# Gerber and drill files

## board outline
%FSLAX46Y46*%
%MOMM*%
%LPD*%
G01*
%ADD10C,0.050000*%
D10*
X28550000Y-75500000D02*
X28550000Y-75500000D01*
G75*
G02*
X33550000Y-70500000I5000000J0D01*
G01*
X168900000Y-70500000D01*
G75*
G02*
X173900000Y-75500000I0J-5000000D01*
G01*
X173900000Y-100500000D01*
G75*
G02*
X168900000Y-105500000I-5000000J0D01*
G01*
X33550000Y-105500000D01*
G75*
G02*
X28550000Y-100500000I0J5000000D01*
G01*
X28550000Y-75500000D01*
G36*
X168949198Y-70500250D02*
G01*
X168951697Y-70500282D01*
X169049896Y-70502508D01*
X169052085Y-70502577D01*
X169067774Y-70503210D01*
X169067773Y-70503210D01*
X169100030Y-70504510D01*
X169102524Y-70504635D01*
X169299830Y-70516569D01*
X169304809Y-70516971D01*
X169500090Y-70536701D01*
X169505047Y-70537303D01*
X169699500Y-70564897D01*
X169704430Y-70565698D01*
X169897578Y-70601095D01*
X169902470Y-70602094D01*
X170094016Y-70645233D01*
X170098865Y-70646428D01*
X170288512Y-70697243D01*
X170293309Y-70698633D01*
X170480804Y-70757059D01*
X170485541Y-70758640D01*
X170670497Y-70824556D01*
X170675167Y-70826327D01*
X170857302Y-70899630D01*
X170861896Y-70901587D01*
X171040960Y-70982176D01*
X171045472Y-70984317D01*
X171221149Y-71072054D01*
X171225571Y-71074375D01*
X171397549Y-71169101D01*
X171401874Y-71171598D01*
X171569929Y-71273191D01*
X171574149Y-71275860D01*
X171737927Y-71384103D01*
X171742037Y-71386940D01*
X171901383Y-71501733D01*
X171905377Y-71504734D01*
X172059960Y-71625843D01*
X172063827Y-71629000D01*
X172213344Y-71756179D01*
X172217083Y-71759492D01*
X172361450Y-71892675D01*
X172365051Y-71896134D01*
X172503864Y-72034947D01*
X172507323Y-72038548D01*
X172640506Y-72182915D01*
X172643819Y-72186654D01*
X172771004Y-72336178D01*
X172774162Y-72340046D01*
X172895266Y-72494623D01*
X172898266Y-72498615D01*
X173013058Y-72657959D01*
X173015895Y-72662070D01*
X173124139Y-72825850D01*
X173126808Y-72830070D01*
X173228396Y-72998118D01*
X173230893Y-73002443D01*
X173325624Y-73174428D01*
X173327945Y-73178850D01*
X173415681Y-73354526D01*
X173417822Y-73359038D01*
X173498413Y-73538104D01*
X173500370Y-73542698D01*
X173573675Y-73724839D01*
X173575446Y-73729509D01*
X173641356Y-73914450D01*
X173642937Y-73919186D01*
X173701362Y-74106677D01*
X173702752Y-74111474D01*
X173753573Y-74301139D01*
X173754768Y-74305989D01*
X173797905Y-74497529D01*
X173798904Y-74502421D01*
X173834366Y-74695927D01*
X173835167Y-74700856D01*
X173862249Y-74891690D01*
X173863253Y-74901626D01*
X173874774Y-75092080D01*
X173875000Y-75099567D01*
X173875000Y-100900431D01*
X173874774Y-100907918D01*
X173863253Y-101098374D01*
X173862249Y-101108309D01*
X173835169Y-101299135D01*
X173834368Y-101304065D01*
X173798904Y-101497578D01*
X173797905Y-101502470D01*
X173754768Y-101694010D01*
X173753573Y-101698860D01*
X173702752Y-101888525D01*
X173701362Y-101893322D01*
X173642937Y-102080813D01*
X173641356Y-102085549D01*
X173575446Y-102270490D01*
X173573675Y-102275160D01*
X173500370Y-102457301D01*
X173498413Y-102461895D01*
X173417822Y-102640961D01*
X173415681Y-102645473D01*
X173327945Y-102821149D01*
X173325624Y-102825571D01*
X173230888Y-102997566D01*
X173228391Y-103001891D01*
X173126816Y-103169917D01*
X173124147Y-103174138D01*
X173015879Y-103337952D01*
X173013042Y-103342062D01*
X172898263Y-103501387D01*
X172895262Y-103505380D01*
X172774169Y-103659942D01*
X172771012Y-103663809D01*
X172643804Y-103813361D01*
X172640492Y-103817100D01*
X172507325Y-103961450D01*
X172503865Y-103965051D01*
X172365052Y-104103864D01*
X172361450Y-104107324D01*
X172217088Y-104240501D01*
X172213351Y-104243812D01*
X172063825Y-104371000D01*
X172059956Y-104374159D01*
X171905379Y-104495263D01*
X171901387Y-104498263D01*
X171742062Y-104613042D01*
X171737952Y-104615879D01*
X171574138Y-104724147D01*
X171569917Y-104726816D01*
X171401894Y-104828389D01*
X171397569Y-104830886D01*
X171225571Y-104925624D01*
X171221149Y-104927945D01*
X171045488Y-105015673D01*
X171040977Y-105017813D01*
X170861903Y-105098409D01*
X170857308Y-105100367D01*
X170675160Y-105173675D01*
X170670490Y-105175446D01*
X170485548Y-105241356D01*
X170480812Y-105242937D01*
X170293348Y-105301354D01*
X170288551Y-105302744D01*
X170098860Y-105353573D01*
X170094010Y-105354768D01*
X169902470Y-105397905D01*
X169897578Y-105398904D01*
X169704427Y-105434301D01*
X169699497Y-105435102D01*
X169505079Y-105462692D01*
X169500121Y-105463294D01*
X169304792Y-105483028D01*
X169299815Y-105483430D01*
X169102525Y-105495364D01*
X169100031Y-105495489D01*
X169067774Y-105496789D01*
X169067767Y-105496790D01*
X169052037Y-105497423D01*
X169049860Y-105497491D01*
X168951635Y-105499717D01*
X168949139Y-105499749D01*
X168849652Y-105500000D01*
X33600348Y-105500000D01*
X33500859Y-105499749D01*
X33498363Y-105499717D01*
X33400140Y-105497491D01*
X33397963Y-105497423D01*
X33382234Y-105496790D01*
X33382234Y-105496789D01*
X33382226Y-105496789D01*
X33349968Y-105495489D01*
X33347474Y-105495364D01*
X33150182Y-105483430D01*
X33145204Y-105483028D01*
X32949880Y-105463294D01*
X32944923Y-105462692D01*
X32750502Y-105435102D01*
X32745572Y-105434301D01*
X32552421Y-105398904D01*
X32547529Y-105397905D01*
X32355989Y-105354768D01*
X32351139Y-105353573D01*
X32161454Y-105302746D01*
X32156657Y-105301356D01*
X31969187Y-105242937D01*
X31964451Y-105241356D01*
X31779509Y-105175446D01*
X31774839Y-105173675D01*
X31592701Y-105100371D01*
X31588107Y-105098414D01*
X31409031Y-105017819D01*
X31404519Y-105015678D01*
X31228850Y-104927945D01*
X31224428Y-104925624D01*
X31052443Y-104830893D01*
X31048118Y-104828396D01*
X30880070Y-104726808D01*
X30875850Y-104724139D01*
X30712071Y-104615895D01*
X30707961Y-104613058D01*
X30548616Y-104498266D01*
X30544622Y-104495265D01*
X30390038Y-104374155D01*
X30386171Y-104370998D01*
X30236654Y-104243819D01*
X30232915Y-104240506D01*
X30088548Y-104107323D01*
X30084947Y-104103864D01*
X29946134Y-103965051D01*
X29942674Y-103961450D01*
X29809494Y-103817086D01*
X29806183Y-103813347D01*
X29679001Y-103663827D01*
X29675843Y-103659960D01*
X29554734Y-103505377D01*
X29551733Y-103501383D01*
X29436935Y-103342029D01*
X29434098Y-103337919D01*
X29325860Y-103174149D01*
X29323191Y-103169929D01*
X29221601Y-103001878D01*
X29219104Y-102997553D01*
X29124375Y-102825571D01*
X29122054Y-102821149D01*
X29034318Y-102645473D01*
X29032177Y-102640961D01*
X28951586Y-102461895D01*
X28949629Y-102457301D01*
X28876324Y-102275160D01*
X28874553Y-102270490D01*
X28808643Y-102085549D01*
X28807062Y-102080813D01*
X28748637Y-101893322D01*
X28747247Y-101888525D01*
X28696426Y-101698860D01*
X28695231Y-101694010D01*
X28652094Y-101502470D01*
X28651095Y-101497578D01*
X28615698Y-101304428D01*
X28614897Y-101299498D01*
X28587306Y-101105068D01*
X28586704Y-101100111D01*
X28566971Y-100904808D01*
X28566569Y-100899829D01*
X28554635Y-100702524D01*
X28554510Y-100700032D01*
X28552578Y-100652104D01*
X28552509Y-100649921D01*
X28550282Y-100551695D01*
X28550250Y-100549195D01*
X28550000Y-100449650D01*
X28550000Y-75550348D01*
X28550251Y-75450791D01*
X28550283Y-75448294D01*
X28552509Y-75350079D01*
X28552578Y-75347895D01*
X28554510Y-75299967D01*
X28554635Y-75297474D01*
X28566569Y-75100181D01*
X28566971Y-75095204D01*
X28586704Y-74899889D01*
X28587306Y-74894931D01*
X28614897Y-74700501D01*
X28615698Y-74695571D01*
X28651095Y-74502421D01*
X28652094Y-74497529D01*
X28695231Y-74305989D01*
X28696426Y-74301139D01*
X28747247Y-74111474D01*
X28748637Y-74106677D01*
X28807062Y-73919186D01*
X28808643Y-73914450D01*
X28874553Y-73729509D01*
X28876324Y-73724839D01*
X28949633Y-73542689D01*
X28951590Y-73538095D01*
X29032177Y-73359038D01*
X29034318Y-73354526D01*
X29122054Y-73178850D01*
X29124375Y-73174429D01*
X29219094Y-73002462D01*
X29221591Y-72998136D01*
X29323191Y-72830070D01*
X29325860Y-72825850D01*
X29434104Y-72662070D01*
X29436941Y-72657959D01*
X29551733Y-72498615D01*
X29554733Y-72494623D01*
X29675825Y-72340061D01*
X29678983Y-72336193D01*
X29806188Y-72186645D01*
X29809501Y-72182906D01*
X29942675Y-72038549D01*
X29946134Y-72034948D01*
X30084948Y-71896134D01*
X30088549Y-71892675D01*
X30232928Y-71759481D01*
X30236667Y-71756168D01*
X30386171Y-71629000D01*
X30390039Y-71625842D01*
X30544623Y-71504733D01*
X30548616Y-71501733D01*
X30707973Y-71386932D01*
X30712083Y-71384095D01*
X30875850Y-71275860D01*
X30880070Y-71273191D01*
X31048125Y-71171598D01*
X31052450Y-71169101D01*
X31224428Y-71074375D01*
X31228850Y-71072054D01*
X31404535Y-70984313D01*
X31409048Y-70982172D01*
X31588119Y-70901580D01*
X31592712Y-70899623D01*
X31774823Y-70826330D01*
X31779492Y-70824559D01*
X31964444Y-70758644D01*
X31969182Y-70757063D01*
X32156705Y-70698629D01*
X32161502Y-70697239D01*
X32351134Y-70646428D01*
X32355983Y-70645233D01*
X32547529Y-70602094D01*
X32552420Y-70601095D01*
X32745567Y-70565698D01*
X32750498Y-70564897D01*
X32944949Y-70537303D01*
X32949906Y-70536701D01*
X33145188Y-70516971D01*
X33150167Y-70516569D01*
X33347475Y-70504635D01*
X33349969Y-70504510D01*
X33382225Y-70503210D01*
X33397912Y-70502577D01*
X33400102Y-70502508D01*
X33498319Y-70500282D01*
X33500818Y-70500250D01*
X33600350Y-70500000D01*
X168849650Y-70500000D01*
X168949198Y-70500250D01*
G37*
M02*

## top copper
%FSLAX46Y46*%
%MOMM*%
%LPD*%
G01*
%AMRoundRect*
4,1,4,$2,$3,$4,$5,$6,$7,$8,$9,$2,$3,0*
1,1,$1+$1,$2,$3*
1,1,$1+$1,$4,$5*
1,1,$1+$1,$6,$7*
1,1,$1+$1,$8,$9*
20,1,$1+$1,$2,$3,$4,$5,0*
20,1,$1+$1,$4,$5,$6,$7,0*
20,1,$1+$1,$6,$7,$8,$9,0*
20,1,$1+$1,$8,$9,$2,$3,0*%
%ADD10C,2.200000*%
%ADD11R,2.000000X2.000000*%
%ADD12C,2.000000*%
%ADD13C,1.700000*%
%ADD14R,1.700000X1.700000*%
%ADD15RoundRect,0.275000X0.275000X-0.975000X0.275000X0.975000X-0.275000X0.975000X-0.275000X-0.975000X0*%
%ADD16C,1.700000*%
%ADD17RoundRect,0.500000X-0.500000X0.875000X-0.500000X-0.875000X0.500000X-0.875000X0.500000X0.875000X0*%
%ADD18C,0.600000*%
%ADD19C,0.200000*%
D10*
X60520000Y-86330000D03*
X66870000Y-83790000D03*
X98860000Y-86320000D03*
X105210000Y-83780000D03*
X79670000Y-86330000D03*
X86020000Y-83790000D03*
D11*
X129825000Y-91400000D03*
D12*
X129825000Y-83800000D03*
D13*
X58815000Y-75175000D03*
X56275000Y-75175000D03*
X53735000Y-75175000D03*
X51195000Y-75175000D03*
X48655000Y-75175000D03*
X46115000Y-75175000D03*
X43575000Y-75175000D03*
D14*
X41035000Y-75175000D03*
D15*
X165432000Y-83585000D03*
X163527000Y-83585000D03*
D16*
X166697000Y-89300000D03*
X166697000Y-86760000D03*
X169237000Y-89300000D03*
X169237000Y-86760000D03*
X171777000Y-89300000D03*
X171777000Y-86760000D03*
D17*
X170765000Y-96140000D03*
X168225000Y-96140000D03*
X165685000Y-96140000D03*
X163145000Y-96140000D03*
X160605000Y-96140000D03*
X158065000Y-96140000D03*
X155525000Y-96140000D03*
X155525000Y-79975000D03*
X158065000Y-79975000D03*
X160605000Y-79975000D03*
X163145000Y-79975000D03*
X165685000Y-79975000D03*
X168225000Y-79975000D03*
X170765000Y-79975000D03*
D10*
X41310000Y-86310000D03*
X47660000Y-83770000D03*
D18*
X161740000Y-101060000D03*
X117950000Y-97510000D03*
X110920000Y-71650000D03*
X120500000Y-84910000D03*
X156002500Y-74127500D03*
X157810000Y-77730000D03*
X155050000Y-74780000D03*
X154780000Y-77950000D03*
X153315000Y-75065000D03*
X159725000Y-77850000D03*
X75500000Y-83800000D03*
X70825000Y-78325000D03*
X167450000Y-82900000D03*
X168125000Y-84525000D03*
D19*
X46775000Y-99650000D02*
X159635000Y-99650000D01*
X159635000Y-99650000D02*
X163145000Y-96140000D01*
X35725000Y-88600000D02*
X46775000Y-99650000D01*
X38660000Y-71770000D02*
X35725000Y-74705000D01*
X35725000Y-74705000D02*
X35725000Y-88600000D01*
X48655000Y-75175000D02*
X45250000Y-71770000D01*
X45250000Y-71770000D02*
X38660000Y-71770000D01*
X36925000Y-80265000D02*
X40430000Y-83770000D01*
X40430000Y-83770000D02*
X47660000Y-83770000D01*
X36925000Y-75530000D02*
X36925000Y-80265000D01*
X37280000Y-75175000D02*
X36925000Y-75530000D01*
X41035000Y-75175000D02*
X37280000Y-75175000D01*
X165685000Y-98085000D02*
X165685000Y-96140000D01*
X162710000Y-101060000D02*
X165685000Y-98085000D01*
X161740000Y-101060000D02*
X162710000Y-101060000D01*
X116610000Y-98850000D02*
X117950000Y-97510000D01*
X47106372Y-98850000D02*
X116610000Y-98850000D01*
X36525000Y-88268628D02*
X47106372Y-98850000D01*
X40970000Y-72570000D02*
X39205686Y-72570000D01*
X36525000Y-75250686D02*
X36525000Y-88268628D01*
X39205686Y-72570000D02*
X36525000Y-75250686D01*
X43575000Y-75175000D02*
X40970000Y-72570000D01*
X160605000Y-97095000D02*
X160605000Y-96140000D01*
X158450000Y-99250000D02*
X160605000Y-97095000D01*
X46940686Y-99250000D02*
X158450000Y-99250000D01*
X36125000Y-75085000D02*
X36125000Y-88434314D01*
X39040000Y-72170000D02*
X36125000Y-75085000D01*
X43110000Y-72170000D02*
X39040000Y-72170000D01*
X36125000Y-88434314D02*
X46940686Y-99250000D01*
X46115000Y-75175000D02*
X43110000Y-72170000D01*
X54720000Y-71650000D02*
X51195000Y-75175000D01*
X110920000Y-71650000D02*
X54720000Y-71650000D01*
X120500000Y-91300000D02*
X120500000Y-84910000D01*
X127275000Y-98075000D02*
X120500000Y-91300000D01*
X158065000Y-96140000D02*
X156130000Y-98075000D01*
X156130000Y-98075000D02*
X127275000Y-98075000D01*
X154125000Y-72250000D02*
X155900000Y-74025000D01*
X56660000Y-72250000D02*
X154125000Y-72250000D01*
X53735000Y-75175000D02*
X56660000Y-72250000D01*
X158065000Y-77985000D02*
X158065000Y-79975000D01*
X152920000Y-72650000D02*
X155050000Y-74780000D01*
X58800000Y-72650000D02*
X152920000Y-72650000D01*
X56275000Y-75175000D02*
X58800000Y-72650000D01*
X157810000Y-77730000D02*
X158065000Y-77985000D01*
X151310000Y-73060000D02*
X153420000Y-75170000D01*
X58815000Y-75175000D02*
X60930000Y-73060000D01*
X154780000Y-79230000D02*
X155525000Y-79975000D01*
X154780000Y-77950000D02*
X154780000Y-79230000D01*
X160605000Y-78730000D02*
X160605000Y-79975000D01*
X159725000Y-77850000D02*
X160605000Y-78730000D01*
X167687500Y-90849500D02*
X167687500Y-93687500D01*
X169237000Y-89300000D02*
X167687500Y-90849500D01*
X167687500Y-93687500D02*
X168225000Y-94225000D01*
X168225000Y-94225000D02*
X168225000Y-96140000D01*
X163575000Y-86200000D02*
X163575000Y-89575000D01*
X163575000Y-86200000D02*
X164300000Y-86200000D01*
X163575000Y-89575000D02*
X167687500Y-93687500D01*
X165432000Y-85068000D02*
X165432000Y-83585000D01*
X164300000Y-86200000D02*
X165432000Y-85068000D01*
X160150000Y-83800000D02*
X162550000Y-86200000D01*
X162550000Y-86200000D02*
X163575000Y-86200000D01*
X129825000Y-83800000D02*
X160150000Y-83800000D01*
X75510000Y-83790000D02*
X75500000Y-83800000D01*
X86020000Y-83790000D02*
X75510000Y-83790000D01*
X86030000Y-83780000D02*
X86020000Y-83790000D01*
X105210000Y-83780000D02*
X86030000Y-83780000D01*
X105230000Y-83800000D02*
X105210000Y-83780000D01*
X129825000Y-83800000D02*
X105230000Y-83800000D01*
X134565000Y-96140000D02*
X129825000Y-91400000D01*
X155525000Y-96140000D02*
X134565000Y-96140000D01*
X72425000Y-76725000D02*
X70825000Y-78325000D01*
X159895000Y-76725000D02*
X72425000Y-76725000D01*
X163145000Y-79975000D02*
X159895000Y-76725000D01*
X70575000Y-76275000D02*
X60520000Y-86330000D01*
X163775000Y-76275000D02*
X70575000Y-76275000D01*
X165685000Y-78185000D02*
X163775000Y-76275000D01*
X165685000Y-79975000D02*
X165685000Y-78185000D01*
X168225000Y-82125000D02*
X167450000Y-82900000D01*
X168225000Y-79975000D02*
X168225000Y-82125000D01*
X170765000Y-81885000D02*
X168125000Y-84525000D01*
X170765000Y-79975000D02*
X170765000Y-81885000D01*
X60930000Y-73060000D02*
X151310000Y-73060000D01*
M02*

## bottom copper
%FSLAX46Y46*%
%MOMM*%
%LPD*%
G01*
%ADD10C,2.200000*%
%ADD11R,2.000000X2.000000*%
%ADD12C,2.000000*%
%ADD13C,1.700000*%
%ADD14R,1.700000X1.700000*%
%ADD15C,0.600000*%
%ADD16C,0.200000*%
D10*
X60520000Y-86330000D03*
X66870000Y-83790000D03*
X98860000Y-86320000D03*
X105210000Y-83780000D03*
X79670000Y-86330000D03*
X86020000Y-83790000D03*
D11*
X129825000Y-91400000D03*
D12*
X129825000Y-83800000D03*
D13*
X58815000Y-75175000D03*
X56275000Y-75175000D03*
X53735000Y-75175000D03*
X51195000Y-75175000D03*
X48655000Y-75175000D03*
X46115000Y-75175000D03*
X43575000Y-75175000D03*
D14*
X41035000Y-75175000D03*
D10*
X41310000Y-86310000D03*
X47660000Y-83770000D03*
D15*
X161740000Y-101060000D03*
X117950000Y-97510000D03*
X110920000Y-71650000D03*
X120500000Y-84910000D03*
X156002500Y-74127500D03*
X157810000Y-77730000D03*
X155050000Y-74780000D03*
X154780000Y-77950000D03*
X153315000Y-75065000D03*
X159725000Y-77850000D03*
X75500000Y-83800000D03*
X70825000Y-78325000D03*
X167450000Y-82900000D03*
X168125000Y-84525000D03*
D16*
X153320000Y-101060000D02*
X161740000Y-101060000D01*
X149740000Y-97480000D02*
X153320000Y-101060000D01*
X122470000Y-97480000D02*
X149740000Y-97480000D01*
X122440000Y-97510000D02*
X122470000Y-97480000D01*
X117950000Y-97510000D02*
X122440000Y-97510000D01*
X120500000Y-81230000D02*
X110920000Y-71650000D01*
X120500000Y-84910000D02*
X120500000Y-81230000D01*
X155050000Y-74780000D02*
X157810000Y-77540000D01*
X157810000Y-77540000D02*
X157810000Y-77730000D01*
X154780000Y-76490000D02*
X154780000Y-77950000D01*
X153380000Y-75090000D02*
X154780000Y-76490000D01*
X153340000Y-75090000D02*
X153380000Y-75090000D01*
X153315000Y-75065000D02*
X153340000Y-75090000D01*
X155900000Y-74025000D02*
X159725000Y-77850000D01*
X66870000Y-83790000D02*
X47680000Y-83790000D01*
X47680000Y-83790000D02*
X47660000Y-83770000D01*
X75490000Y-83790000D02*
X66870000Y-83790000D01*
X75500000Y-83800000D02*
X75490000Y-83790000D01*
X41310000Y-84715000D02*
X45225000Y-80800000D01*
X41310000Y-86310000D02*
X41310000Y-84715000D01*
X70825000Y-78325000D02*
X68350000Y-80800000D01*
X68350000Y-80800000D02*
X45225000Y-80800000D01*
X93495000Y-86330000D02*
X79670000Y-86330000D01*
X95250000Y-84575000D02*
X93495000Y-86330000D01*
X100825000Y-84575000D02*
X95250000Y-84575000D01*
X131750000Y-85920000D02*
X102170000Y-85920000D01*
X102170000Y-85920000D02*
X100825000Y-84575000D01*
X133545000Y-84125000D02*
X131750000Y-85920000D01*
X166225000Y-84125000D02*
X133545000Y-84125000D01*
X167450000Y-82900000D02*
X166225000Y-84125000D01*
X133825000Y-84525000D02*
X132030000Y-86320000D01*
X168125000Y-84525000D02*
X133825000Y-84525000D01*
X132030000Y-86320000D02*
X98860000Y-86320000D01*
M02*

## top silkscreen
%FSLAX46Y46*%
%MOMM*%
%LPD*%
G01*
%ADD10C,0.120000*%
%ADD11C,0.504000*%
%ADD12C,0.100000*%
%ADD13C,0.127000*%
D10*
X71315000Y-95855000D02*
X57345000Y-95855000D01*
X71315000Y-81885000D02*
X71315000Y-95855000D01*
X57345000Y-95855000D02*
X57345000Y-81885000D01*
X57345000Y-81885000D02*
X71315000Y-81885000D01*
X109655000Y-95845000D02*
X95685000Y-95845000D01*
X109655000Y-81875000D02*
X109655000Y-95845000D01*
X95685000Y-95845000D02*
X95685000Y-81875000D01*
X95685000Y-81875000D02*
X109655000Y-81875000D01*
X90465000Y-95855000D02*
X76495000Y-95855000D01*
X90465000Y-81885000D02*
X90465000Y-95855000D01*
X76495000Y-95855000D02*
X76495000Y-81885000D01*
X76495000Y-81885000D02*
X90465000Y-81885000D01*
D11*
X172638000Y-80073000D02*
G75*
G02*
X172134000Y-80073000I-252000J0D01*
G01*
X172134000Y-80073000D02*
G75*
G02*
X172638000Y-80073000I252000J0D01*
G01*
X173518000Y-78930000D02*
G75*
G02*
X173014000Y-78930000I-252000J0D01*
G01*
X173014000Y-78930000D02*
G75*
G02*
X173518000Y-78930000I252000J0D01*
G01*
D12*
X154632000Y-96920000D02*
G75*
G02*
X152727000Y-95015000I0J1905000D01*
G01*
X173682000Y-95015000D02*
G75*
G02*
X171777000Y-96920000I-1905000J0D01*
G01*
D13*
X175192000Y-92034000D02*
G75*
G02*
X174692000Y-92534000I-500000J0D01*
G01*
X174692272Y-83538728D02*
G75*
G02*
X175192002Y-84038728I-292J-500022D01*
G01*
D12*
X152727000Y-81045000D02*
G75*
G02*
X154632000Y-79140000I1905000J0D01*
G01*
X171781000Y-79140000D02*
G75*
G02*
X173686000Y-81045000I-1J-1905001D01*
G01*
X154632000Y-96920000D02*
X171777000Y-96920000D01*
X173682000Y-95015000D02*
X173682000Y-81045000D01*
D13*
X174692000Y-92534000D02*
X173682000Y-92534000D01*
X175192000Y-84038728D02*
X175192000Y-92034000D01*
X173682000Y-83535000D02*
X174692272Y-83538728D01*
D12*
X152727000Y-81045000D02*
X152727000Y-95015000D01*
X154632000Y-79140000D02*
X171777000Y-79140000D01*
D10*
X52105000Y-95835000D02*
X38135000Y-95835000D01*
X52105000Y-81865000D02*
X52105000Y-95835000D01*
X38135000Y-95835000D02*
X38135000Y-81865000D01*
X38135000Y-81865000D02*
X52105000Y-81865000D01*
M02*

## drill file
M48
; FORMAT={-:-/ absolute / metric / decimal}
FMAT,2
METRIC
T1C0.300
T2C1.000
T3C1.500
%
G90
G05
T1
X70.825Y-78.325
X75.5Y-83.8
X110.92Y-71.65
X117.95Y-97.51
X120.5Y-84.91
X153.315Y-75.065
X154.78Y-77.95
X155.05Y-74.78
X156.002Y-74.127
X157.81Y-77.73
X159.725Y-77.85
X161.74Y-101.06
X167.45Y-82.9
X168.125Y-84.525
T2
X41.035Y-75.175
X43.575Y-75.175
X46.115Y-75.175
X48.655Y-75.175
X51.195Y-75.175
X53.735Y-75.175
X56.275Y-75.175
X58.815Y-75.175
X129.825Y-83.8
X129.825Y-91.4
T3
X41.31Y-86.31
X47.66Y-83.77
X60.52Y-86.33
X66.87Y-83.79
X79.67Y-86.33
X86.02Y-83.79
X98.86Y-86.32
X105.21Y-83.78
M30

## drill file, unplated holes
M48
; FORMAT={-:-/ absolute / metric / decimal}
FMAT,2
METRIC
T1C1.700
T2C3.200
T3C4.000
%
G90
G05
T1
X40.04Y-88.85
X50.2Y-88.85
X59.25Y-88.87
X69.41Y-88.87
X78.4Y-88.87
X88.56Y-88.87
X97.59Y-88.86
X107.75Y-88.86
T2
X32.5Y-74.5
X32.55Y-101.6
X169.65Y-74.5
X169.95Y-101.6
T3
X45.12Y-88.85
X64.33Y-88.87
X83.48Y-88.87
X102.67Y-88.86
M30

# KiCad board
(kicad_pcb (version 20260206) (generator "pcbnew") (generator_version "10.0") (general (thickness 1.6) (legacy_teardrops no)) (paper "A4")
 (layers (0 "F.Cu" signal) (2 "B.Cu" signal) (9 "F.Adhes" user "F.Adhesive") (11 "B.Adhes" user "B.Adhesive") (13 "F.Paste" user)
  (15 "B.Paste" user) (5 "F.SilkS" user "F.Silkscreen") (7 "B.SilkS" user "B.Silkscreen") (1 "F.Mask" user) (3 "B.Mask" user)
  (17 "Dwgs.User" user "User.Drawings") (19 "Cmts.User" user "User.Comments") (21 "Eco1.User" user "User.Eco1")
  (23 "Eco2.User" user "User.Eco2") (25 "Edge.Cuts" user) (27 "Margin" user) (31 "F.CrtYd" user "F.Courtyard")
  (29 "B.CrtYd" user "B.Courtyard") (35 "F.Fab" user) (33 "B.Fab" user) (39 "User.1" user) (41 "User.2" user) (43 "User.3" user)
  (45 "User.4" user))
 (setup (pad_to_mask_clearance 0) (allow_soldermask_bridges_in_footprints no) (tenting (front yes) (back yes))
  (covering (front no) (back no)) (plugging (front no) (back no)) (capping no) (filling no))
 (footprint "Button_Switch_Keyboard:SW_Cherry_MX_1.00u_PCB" (layer "F.Cu") (at 86.02 83.79)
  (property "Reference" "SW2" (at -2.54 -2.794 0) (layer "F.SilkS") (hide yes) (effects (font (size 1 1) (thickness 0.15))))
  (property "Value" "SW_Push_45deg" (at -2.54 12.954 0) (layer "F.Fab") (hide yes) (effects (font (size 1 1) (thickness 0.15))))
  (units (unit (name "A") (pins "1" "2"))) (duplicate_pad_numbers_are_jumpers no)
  (fp_line (start -9.525 -1.905) (end 4.445 -1.905) (stroke (width 0.12) (type solid)) (layer "F.SilkS"))
  (fp_line (start -9.525 12.065) (end -9.525 -1.905) (stroke (width 0.12) (type solid)) (layer "F.SilkS"))
  (fp_line (start 4.445 -1.905) (end 4.445 12.065) (stroke (width 0.12) (type solid)) (layer "F.SilkS"))
  (fp_line (start 4.445 12.065) (end -9.525 12.065) (stroke (width 0.12) (type solid)) (layer "F.SilkS"))
  (pad "" np_thru_hole circle (at -7.62 5.08) (size 1.7 1.7) (drill 1.7) (layers "*.Cu" "*.Mask"))
  (pad "" np_thru_hole circle (at -2.54 5.08) (size 4 4) (drill 4) (layers "*.Cu" "*.Mask"))
  (pad "" np_thru_hole circle (at 2.54 5.08) (size 1.7 1.7) (drill 1.7) (layers "*.Cu" "*.Mask"))
  (pad "1" thru_hole circle (at 0 0) (size 2.2 2.2) (drill 1.5) (layers "*.Cu" "*.Mask") (remove_unused_layers no) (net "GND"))
  (pad "2" thru_hole circle (at -6.35 2.54) (size 2.2 2.2) (drill 1.5) (layers "*.Cu" "*.Mask") (remove_unused_layers no)
   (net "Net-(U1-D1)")))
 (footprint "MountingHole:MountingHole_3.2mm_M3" (layer "F.Cu") (at 32.55 101.6)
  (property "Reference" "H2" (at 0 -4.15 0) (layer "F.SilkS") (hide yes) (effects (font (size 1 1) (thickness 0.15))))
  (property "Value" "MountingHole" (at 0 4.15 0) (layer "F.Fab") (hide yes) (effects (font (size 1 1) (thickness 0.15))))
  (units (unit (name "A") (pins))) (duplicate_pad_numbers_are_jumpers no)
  (pad "" np_thru_hole circle (at 0 0) (size 3.2 3.2) (drill 3.2) (layers "*.Cu" "*.Mask")))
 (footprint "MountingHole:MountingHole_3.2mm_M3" (layer "F.Cu") (at 32.5 74.5)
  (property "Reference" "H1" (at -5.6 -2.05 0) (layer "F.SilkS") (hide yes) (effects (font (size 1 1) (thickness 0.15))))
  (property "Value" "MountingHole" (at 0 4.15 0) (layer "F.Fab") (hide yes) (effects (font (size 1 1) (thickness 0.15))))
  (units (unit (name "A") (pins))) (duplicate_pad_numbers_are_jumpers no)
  (pad "" np_thru_hole circle (at 0 0) (size 3.2 3.2) (drill 3.2) (layers "*.Cu" "*.Mask")))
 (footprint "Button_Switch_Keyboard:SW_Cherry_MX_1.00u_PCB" (layer "F.Cu") (at 105.21 83.78)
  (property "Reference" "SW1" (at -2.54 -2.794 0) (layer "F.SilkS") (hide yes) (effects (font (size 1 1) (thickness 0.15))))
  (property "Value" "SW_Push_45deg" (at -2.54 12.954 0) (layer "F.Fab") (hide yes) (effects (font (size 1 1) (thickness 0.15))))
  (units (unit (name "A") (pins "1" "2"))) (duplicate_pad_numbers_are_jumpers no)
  (fp_line (start -9.525 -1.905) (end 4.445 -1.905) (stroke (width 0.12) (type solid)) (layer "F.SilkS"))
  (fp_line (start -9.525 12.065) (end -9.525 -1.905) (stroke (width 0.12) (type solid)) (layer "F.SilkS"))
  (fp_line (start 4.445 -1.905) (end 4.445 12.065) (stroke (width 0.12) (type solid)) (layer "F.SilkS"))
  (fp_line (start 4.445 12.065) (end -9.525 12.065) (stroke (width 0.12) (type solid)) (layer "F.SilkS"))
  (pad "" np_thru_hole circle (at -7.62 5.08) (size 1.7 1.7) (drill 1.7) (layers "*.Cu" "*.Mask"))
  (pad "" np_thru_hole circle (at -2.54 5.08) (size 4 4) (drill 4) (layers "*.Cu" "*.Mask"))
  (pad "" np_thru_hole circle (at 2.54 5.08) (size 1.7 1.7) (drill 1.7) (layers "*.Cu" "*.Mask"))
  (pad "1" thru_hole circle (at 0 0) (size 2.2 2.2) (drill 1.5) (layers "*.Cu" "*.Mask") (remove_unused_layers no) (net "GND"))
  (pad "2" thru_hole circle (at -6.35 2.54) (size 2.2 2.2) (drill 1.5) (layers "*.Cu" "*.Mask") (remove_unused_layers no)
   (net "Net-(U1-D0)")))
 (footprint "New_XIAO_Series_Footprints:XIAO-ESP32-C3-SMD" (layer "F.Cu") (at 152.645 79.14 -90)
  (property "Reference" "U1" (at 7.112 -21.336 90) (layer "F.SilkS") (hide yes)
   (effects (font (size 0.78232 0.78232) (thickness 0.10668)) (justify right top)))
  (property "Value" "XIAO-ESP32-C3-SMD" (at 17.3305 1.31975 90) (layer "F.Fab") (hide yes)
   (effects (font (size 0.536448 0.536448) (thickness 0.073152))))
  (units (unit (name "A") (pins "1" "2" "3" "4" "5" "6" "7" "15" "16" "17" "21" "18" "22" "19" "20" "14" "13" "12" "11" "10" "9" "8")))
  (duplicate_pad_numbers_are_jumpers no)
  (fp_line (start 1.905 -0.082) (end 15.875 -0.082) (stroke (width 0.1) (type solid)) (layer "F.SilkS"))
  (fp_line (start 0 -1.987) (end 0 -19.132) (stroke (width 0.1) (type solid)) (layer "F.SilkS"))
  (fp_line (start 17.78 -1.987) (end 17.78 -19.132) (stroke (width 0.1) (type solid)) (layer "F.SilkS"))
  (fp_line (start 4.395 -21.037) (end 4.398728 -22.047272) (stroke (width 0.127) (type solid)) (layer "F.SilkS"))
  (fp_line (start 15.875 -21.037) (end 1.905 -21.037) (stroke (width 0.1) (type solid)) (layer "F.SilkS"))
  (fp_line (start 13.394 -22.047) (end 13.394 -21.037) (stroke (width 0.127) (type solid)) (layer "F.SilkS"))
  (fp_line (start 4.898728 -22.547) (end 12.894 -22.547) (stroke (width 0.127) (type solid)) (layer "F.SilkS"))
  (fp_arc (start 1.905 -0.082) (mid 0.557962 -0.639962) (end 0 -1.987) (stroke (width 0.1) (type solid)) (layer "F.SilkS"))
  (fp_arc (start 17.78 -1.987) (mid 17.222038 -0.639962) (end 15.875 -0.082) (stroke (width 0.1) (type solid)) (layer "F.SilkS"))
  (fp_arc (start 0 -19.136) (mid 0.557962 -20.483038) (end 1.905 -21.041) (stroke (width 0.1) (type solid)) (layer "F.SilkS"))
  (fp_arc (start 15.875 -21.037) (mid 17.222038 -20.479038) (end 17.78 -19.132) (stroke (width 0.1) (type solid)) (layer "F.SilkS"))
  (fp_arc (start 4.398728 -22.047272) (mid 4.545272 -22.40064) (end 4.898728 -22.547) (stroke (width 0.127) (type default))
   (layer "F.SilkS"))
  (fp_arc (start 12.894 -22.547) (mid 13.247553 -22.400553) (end 13.394 -22.047) (stroke (width 0.127) (type default)) (layer "F.SilkS"))
  (fp_circle (center 0.933 -19.741) (end 0.933 -19.995) (stroke (width 0.5) (type solid)) (fill yes) (layer "F.SilkS"))
  (fp_circle (center -0.21 -20.621) (end -0.21 -20.875) (stroke (width 0.5) (type solid)) (fill yes) (layer "F.SilkS"))
  (pad "1" smd roundrect (at 0.835 -18.12 270) (size 2.75 2) (layers "F.Cu" "F.Mask" "F.Paste") (roundrect_rratio 0.25) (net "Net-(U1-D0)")
   (solder_mask_margin 0.0508) (thermal_bridge_angle 45))
  (pad "2" smd roundrect (at 0.835 -15.58 270) (size 2.75 2) (layers "F.Cu" "F.Mask" "F.Paste") (roundrect_rratio 0.25) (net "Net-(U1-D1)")
   (solder_mask_margin 0.0508) (thermal_bridge_angle 45))
  (pad "3" smd roundrect (at 0.835 -13.04 270) (size 2.75 2) (layers "F.Cu" "F.Mask" "F.Paste") (roundrect_rratio 0.25) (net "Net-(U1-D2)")
   (solder_mask_margin 0.0508) (thermal_bridge_angle 45))
  (pad "4" smd roundrect (at 0.835 -10.5 270) (size 2.75 2) (layers "F.Cu" "F.Mask" "F.Paste") (roundrect_rratio 0.25) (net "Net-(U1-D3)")
   (solder_mask_margin 0.0508) (thermal_bridge_angle 45))
  (pad "5" smd roundrect (at 0.835 -7.96 270) (size 2.75 2) (layers "F.Cu" "F.Mask" "F.Paste") (roundrect_rratio 0.25) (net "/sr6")
   (solder_mask_margin 0.0508) (thermal_bridge_angle 45))
  (pad "6" smd roundrect (at 0.835 -5.42 270) (size 2.75 2) (layers "F.Cu" "F.Mask" "F.Paste") (roundrect_rratio 0.25) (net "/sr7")
   (solder_mask_margin 0.0508) (thermal_bridge_angle 45))
  (pad "7" smd roundrect (at 0.835 -2.88 270) (size 2.75 2) (layers "F.Cu" "F.Mask" "F.Paste") (roundrect_rratio 0.25) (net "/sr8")
   (solder_mask_margin 0.0508) (thermal_bridge_angle 45))
  (pad "8" smd roundrect (at 17 -2.88 270) (size 2.75 2) (layers "F.Cu" "F.Mask" "F.Paste") (roundrect_rratio 0.25) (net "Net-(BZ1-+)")
   (solder_mask_margin 0.0508) (thermal_bridge_angle 45))
  (pad "9" smd roundrect (at 17 -5.42 270) (size 2.75 2) (layers "F.Cu" "F.Mask" "F.Paste") (roundrect_rratio 0.25) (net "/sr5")
   (solder_mask_margin 0.0508) (thermal_bridge_angle 45))
  (pad "10" smd roundrect (at 17 -7.96 270) (size 2.75 2) (layers "F.Cu" "F.Mask" "F.Paste") (roundrect_rratio 0.25) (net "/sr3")
   (solder_mask_margin 0.0508) (thermal_bridge_angle 45))
  (pad "11" smd roundrect (at 17 -10.5 270) (size 2.75 2) (layers "F.Cu" "F.Mask" "F.Paste") (roundrect_rratio 0.25) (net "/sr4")
   (solder_mask_margin 0.0508) (thermal_bridge_angle 45))
  (pad "12" smd roundrect (at 17 -13.04 270) (size 2.75 2) (layers "F.Cu" "F.Mask" "F.Paste") (roundrect_rratio 0.25) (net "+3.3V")
   (solder_mask_margin 0.0508) (thermal_bridge_angle 45))
  (pad "13" smd roundrect (at 17 -15.58 270) (size 2.75 2) (layers "F.Cu" "F.Mask" "F.Paste") (roundrect_rratio 0.25) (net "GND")
   (solder_mask_margin 0.0508) (thermal_bridge_angle 45))
  (pad "14" smd roundrect (at 17 -18.12 270) (size 2.75 2) (layers "F.Cu" "F.Mask" "F.Paste") (roundrect_rratio 0.25)
   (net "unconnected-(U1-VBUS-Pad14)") (solder_mask_margin 0.0508) (thermal_bridge_angle 45))
  (pad "15" smd circle (at 7.62 -19.132 270) (size 1.7 1.7) (layers "F.Cu" "F.Mask" "F.Paste") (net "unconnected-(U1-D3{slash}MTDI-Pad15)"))
  (pad "16" smd circle (at 10.16 -19.132 270) (size 1.7 1.7) (layers "F.Cu" "F.Mask" "F.Paste") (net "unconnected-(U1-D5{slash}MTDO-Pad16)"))
  (pad "17" smd circle (at 7.62 -16.592 270) (size 1.7 1.7) (layers "F.Cu" "F.Mask" "F.Paste") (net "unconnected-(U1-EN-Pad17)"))
  (pad "18" smd circle (at 10.16 -16.592 270) (size 1.7 1.7) (layers "F.Cu" "F.Mask" "F.Paste") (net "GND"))
  (pad "19" smd circle (at 7.62 -14.052 270) (size 1.7 1.7) (layers "F.Cu" "F.Mask" "F.Paste") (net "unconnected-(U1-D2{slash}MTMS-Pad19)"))
  (pad "20" smd circle (at 10.16 -14.052 270) (size 1.7 1.7) (layers "F.Cu" "F.Mask" "F.Paste") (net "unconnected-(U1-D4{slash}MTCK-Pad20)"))
  (pad "21" smd roundrect (at 4.445 -10.882 90) (size 2.5 1.1) (layers "F.Cu" "F.Mask" "F.Paste") (roundrect_rratio 0.25)
   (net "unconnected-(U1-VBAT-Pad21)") (thermal_bridge_angle 45))
  (pad "22" smd roundrect (at 4.445 -12.787 90) (size 2.5 1.1) (layers "F.Cu" "F.Mask" "F.Paste") (roundrect_rratio 0.25) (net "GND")
   (thermal_bridge_angle 45)))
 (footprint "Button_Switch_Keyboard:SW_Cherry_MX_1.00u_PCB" (layer "F.Cu") (at 47.66 83.77)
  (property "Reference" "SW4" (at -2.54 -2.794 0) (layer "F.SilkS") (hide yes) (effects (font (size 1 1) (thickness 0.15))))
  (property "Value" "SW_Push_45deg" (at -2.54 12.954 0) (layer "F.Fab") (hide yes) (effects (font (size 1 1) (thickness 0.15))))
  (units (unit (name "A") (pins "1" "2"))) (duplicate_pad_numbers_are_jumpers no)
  (fp_line (start -9.525 -1.905) (end 4.445 -1.905) (stroke (width 0.12) (type solid)) (layer "F.SilkS"))
  (fp_line (start -9.525 12.065) (end -9.525 -1.905) (stroke (width 0.12) (type solid)) (layer "F.SilkS"))
  (fp_line (start 4.445 -1.905) (end 4.445 12.065) (stroke (width 0.12) (type solid)) (layer "F.SilkS"))
  (fp_line (start 4.445 12.065) (end -9.525 12.065) (stroke (width 0.12) (type solid)) (layer "F.SilkS"))
  (pad "" np_thru_hole circle (at -7.62 5.08) (size 1.7 1.7) (drill 1.7) (layers "*.Cu" "*.Mask"))
  (pad "" np_thru_hole circle (at -2.54 5.08) (size 4 4) (drill 4) (layers "*.Cu" "*.Mask"))
  (pad "" np_thru_hole circle (at 2.54 5.08) (size 1.7 1.7) (drill 1.7) (layers "*.Cu" "*.Mask"))
  (pad "1" thru_hole circle (at 0 0) (size 2.2 2.2) (drill 1.5) (layers "*.Cu" "*.Mask") (remove_unused_layers no) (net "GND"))
  (pad "2" thru_hole circle (at -6.35 2.54) (size 2.2 2.2) (drill 1.5) (layers "*.Cu" "*.Mask") (remove_unused_layers no)
   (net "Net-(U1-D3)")))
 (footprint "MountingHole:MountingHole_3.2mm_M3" (layer "F.Cu") (at 169.65 74.5)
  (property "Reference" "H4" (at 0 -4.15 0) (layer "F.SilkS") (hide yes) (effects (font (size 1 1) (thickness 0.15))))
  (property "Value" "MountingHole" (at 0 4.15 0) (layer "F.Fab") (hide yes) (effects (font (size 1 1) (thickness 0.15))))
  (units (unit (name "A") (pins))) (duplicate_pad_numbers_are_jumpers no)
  (pad "" np_thru_hole circle (at 0 0) (size 3.2 3.2) (drill 3.2) (layers "*.Cu" "*.Mask")))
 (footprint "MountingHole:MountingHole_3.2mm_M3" (layer "F.Cu") (at 169.95 101.6)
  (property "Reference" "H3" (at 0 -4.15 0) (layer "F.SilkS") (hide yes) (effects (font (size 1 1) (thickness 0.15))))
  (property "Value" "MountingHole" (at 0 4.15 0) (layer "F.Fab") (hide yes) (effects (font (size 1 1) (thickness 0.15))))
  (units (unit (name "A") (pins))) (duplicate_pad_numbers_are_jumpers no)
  (pad "" np_thru_hole circle (at 0 0) (size 3.2 3.2) (drill 3.2) (layers "*.Cu" "*.Mask")))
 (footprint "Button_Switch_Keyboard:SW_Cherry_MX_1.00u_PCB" (layer "F.Cu") (at 66.87 83.79)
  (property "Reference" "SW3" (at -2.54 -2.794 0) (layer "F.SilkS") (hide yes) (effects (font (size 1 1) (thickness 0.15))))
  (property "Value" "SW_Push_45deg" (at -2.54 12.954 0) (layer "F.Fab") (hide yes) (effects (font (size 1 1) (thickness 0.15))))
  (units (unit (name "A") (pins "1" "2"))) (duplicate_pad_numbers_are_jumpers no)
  (fp_line (start -9.525 -1.905) (end 4.445 -1.905) (stroke (width 0.12) (type solid)) (layer "F.SilkS"))
  (fp_line (start -9.525 12.065) (end -9.525 -1.905) (stroke (width 0.12) (type solid)) (layer "F.SilkS"))
  (fp_line (start 4.445 -1.905) (end 4.445 12.065) (stroke (width 0.12) (type solid)) (layer "F.SilkS"))
  (fp_line (start 4.445 12.065) (end -9.525 12.065) (stroke (width 0.12) (type solid)) (layer "F.SilkS"))
  (pad "" np_thru_hole circle (at -7.62 5.08) (size 1.7 1.7) (drill 1.7) (layers "*.Cu" "*.Mask"))
  (pad "" np_thru_hole circle (at -2.54 5.08) (size 4 4) (drill 4) (layers "*.Cu" "*.Mask"))
  (pad "" np_thru_hole circle (at 2.54 5.08) (size 1.7 1.7) (drill 1.7) (layers "*.Cu" "*.Mask"))
  (pad "1" thru_hole circle (at 0 0) (size 2.2 2.2) (drill 1.5) (layers "*.Cu" "*.Mask") (remove_unused_layers no) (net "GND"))
  (pad "2" thru_hole circle (at -6.35 2.54) (size 2.2 2.2) (drill 1.5) (layers "*.Cu" "*.Mask") (remove_unused_layers no)
   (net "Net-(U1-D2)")))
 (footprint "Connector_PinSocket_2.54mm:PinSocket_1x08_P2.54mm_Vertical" (layer "B.Cu") (at 41.035 75.175 -90)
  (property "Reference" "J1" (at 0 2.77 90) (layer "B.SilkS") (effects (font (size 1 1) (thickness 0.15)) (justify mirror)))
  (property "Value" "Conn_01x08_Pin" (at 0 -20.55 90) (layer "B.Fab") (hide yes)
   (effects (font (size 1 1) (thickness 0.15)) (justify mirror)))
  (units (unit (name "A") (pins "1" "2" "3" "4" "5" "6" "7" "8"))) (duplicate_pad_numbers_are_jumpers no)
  (pad "1" thru_hole rect (at 0 0 270) (size 1.7 1.7) (drill 1) (layers "*.Cu" "*.Mask") (remove_unused_layers no) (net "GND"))
  (pad "2" thru_hole circle (at 0 -2.54 270) (size 1.7 1.7) (drill 1) (layers "*.Cu" "*.Mask") (remove_unused_layers no) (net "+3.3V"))
  (pad "3" thru_hole circle (at 0 -5.08 270) (size 1.7 1.7) (drill 1) (layers "*.Cu" "*.Mask") (remove_unused_layers no) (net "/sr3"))
  (pad "4" thru_hole circle (at 0 -7.62 270) (size 1.7 1.7) (drill 1) (layers "*.Cu" "*.Mask") (remove_unused_layers no) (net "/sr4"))
  (pad "5" thru_hole circle (at 0 -10.16 270) (size 1.7 1.7) (drill 1) (layers "*.Cu" "*.Mask") (remove_unused_layers no) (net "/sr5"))
  (pad "6" thru_hole circle (at 0 -12.7 270) (size 1.7 1.7) (drill 1) (layers "*.Cu" "*.Mask") (remove_unused_layers no) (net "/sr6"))
  (pad "7" thru_hole circle (at 0 -15.24 270) (size 1.7 1.7) (drill 1) (layers "*.Cu" "*.Mask") (remove_unused_layers no) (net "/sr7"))
  (pad "8" thru_hole circle (at 0 -17.78 270) (size 1.7 1.7) (drill 1) (layers "*.Cu" "*.Mask") (remove_unused_layers no) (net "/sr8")))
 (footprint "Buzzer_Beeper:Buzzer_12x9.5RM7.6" (layer "B.Cu") (at 129.825 91.4 90)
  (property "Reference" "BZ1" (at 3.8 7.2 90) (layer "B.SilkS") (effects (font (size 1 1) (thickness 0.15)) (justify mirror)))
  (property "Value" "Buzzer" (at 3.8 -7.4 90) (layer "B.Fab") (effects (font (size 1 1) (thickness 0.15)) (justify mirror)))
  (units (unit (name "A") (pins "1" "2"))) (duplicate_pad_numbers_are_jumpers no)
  (pad "1" thru_hole rect (at 0 0 90) (size 2 2) (drill 1) (layers "*.Cu" "*.Mask") (remove_unused_layers no) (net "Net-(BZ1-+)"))
  (pad "2" thru_hole circle (at 7.6 0 90) (size 2 2) (drill 1) (layers "*.Cu" "*.Mask") (remove_unused_layers no) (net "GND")))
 (gr_rect (start 28.55 70.5) (end 173.9 105.5) (radius 5) (stroke (width 0.05) (type solid)) (fill no) (layer "Edge.Cuts"))
 (segment (start 167.6875 90.8495) (end 167.6875 93.6875) (width 0.2) (layer "F.Cu") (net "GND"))
 (segment (start 129.825 83.8) (end 105.23 83.8) (width 0.2) (layer "F.Cu") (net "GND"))
 (segment (start 162.55 86.2) (end 163.575 86.2) (width 0.2) (layer "F.Cu") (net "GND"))
 (segment (start 163.575 89.575) (end 167.6875 93.6875) (width 0.2) (layer "F.Cu") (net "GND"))
 (segment (start 86.03 83.78) (end 86.02 83.79) (width 0.2) (layer "F.Cu") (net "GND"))
 (segment (start 168.225 94.225) (end 168.225 96.14) (width 0.2) (layer "F.Cu") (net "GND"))
 (segment (start 86.02 83.79) (end 75.51 83.79) (width 0.2) (layer "F.Cu") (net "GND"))
 (segment (start 163.575 86.2) (end 163.575 89.575) (width 0.2) (layer "F.Cu") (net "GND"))
 (segment (start 169.237 89.3) (end 167.6875 90.8495) (width 0.2) (layer "F.Cu") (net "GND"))
 (segment (start 165.432 85.068) (end 165.432 83.585) (width 0.2) (layer "F.Cu") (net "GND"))
 (segment (start 160.15 83.8) (end 162.55 86.2) (width 0.2) (layer "F.Cu") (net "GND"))
 (segment (start 36.925 75.53) (end 36.925 80.265) (width 0.2) (layer "F.Cu") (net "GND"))
 (segment (start 75.51 83.79) (end 75.5 83.8) (width 0.2) (layer "F.Cu") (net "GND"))
 (segment (start 40.43 83.77) (end 47.66 83.77) (width 0.2) (layer "F.Cu") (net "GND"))
 (segment (start 36.925 80.265) (end 40.43 83.77) (width 0.2) (layer "F.Cu") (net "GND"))
 (segment (start 129.825 83.8) (end 160.15 83.8) (width 0.2) (layer "F.Cu") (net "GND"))
 (segment (start 41.035 75.175) (end 37.28 75.175) (width 0.2) (layer "F.Cu") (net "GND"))
 (segment (start 167.6875 93.6875) (end 168.225 94.225) (width 0.2) (layer "F.Cu") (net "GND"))
 (segment (start 37.28 75.175) (end 36.925 75.53) (width 0.2) (layer "F.Cu") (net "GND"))
 (segment (start 105.21 83.78) (end 86.03 83.78) (width 0.2) (layer "F.Cu") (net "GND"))
 (segment (start 164.3 86.2) (end 165.432 85.068) (width 0.2) (layer "F.Cu") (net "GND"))
 (segment (start 163.575 86.2) (end 164.3 86.2) (width 0.2) (layer "F.Cu") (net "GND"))
 (segment (start 105.23 83.8) (end 105.21 83.78) (width 0.2) (layer "F.Cu") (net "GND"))
 (via (at 75.5 83.8) (size 0.6) (drill 0.3) (layers "F.Cu" "B.Cu") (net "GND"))
 (segment (start 75.5 83.8) (end 75.49 83.79) (width 0.2) (layer "B.Cu") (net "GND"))
 (segment (start 47.68 83.79) (end 47.66 83.77) (width 0.2) (layer "B.Cu") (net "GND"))
 (segment (start 75.49 83.79) (end 66.87 83.79) (width 0.2) (layer "B.Cu") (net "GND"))
 (segment (start 66.87 83.79) (end 47.68 83.79) (width 0.2) (layer "B.Cu") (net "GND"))
 (segment (start 134.565 96.14) (end 129.825 91.4) (width 0.2) (layer "F.Cu") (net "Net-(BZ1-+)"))
 (segment (start 155.525 96.14) (end 134.565 96.14) (width 0.2) (layer "F.Cu") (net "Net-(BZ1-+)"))
 (segment (start 160.605 78.73) (end 160.605 79.975) (width 0.2) (layer "F.Cu") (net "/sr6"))
 (segment (start 56.66 72.25) (end 154.125 72.25) (width 0.2) (layer "F.Cu") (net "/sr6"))
 (segment (start 154.125 72.25) (end 155.9 74.025) (width 0.2) (layer "F.Cu") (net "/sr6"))
 (segment (start 53.735 75.175) (end 56.66 72.25) (width 0.2) (layer "F.Cu") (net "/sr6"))
 (segment (start 159.725 77.85) (end 160.605 78.73) (width 0.2) (layer "F.Cu") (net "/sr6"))
 (via (at 159.725 77.85) (size 0.6) (drill 0.3) (layers "F.Cu" "B.Cu") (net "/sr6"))
 (via (at 156.0025 74.1275) (size 0.6) (drill 0.3) (layers "F.Cu" "B.Cu") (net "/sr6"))
 (segment (start 155.9 74.025) (end 159.725 77.85) (width 0.2) (layer "B.Cu") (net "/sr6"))
 (segment (start 151.31 73.06) (end 153.42 75.17) (width 0.2) (layer "F.Cu") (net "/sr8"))
 (segment (start 154.78 79.23) (end 155.525 79.975) (width 0.2) (layer "F.Cu") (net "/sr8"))
 (segment (start 58.815 75.175) (end 60.93 73.06) (width 0.2) (layer "F.Cu") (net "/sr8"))
 (segment (start 60.93 73.06) (end 151.31 73.06) (width 0.2) (layer "F.Cu") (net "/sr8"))
 (segment (start 154.78 77.95) (end 154.78 79.23) (width 0.2) (layer "F.Cu") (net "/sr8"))
 (via (at 154.78 77.95) (size 0.6) (drill 0.3) (layers "F.Cu" "B.Cu") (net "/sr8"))
 (via (at 153.315 75.065) (size 0.6) (drill 0.3) (layers "F.Cu" "B.Cu") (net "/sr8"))
 (segment (start 153.34 75.09) (end 153.38 75.09) (width 0.2) (layer "B.Cu") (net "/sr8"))
 (segment (start 153.38 75.09) (end 154.78 76.49) (width 0.2) (layer "B.Cu") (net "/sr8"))
 (segment (start 153.315 75.065) (end 153.34 75.09) (width 0.2) (layer "B.Cu") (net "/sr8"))
 (segment (start 154.78 76.49) (end 154.78 77.95) (width 0.2) (layer "B.Cu") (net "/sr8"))
 (segment (start 127.275 98.075) (end 120.5 91.3) (width 0.2) (layer "F.Cu") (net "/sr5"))
 (segment (start 110.92 71.65) (end 54.72 71.65) (width 0.2) (layer "F.Cu") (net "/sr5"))
 (segment (start 54.72 71.65) (end 51.195 75.175) (width 0.2) (layer "F.Cu") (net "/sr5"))
 (segment (start 158.065 96.14) (end 156.13 98.075) (width 0.2) (layer "F.Cu") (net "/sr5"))
 (segment (start 156.13 98.075) (end 127.275 98.075) (width 0.2) (layer "F.Cu") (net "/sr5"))
 (segment (start 120.5 91.3) (end 120.5 84.91) (width 0.2) (layer "F.Cu") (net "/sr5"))
 (via (at 110.92 71.65) (size 0.6) (drill 0.3) (layers "F.Cu" "B.Cu") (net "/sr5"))
 (via (at 120.5 84.91) (size 0.6) (drill 0.3) (layers "F.Cu" "B.Cu") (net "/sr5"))
 (segment (start 120.5 81.23) (end 110.92 71.65) (width 0.2) (layer "B.Cu") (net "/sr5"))
 (segment (start 120.5 84.91) (end 120.5 81.23) (width 0.2) (layer "B.Cu") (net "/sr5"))
 (segment (start 43.575 75.175) (end 40.97 72.57) (width 0.2) (layer "F.Cu") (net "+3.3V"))
 (segment (start 165.685 98.085) (end 165.685 96.14) (width 0.2) (layer "F.Cu") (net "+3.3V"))
 (segment (start 36.525 88.268628) (end 47.106372 98.85) (width 0.2) (layer "F.Cu") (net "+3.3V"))
 (segment (start 40.97 72.57) (end 39.205686 72.57) (width 0.2) (layer "F.Cu") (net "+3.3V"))
 (segment (start 161.74 101.06) (end 162.71 101.06) (width 0.2) (layer "F.Cu") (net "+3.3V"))
 (segment (start 162.71 101.06) (end 165.685 98.085) (width 0.2) (layer "F.Cu") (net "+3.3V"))
 (segment (start 116.61 98.85) (end 117.95 97.51) (width 0.2) (layer "F.Cu") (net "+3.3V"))
 (segment (start 47.106372 98.85) (end 116.61 98.85) (width 0.2) (layer "F.Cu") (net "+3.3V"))
 (segment (start 39.205686 72.57) (end 36.525 75.250686) (width 0.2) (layer "F.Cu") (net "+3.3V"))
 (segment (start 36.525 75.250686) (end 36.525 88.268628) (width 0.2) (layer "F.Cu") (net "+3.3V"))
 (via (at 161.74 101.06) (size 0.6) (drill 0.3) (layers "F.Cu" "B.Cu") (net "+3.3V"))
 (via (at 117.95 97.51) (size 0.6) (drill 0.3) (layers "F.Cu" "B.Cu") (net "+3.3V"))
 (segment (start 122.47 97.48) (end 149.74 97.48) (width 0.2) (layer "B.Cu") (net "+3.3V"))
 (segment (start 122.44 97.51) (end 122.47 97.48) (width 0.2) (layer "B.Cu") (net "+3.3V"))
 (segment (start 149.74 97.48) (end 153.32 101.06) (width 0.2) (layer "B.Cu") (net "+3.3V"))
 (segment (start 117.95 97.51) (end 122.44 97.51) (width 0.2) (layer "B.Cu") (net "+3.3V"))
 (segment (start 153.32 101.06) (end 161.74 101.06) (width 0.2) (layer "B.Cu") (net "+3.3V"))
 (segment (start 36.125 75.085) (end 36.125 88.434314) (width 0.2) (layer "F.Cu") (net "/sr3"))
 (segment (start 160.605 97.095) (end 160.605 96.14) (width 0.2) (layer "F.Cu") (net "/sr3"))
 (segment (start 36.125 88.434314) (end 46.940686 99.25) (width 0.2) (layer "F.Cu") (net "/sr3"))
 (segment (start 43.11 72.17) (end 39.04 72.17) (width 0.2) (layer "F.Cu") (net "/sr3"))
 (segment (start 46.940686 99.25) (end 158.45 99.25) (width 0.2) (layer "F.Cu") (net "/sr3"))
 (segment (start 158.45 99.25) (end 160.605 97.095) (width 0.2) (layer "F.Cu") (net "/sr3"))
 (segment (start 46.115 75.175) (end 43.11 72.17) (width 0.2) (layer "F.Cu") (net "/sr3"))
 (segment (start 39.04 72.17) (end 36.125 75.085) (width 0.2) (layer "F.Cu") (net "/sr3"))
 (segment (start 157.81 77.73) (end 158.065 77.985) (width 0.2) (layer "F.Cu") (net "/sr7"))
 (segment (start 56.275 75.175) (end 58.8 72.65) (width 0.2) (layer "F.Cu") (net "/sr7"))
 (segment (start 58.8 72.65) (end 152.92 72.65) (width 0.2) (layer "F.Cu") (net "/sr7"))
 (segment (start 158.065 77.985) (end 158.065 79.975) (width 0.2) (layer "F.Cu") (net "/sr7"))
 (segment (start 152.92 72.65) (end 155.05 74.78) (width 0.2) (layer "F.Cu") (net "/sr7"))
 (via (at 155.05 74.78) (size 0.6) (drill 0.3) (layers "F.Cu" "B.Cu") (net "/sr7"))
 (via (at 157.81 77.73) (size 0.6) (drill 0.3) (layers "F.Cu" "B.Cu") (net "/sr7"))
 (segment (start 155.05 74.78) (end 157.81 77.54) (width 0.2) (layer "B.Cu") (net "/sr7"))
 (segment (start 157.81 77.54) (end 157.81 77.73) (width 0.2) (layer "B.Cu") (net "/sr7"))
 (segment (start 159.635 99.65) (end 163.145 96.14) (width 0.2) (layer "F.Cu") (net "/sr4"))
 (segment (start 45.25 71.77) (end 38.66 71.77) (width 0.2) (layer "F.Cu") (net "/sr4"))
 (segment (start 46.775 99.65) (end 159.635 99.65) (width 0.2) (layer "F.Cu") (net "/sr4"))
 (segment (start 38.66 71.77) (end 35.725 74.705) (width 0.2) (layer "F.Cu") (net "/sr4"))
 (segment (start 35.725 74.705) (end 35.725 88.6) (width 0.2) (layer "F.Cu") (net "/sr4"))
 (segment (start 48.655 75.175) (end 45.25 71.77) (width 0.2) (layer "F.Cu") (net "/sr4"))
 (segment (start 35.725 88.6) (end 46.775 99.65) (width 0.2) (layer "F.Cu") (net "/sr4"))
 (segment (start 170.765 79.975) (end 170.765 81.885) (width 0.2) (layer "F.Cu") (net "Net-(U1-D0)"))
 (segment (start 170.765 81.885) (end 168.125 84.525) (width 0.2) (layer "F.Cu") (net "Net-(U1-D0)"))
 (via (at 168.125 84.525) (size 0.6) (drill 0.3) (layers "F.Cu" "B.Cu") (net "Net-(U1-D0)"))
 (segment (start 132.03 86.32) (end 98.86 86.32) (width 0.2) (layer "B.Cu") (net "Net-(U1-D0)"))
 (segment (start 168.125 84.525) (end 133.825 84.525) (width 0.2) (layer "B.Cu") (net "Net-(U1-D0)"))
 (segment (start 133.825 84.525) (end 132.03 86.32) (width 0.2) (layer "B.Cu") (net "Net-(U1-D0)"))
 (segment (start 168.225 82.125) (end 167.45 82.9) (width 0.2) (layer "F.Cu") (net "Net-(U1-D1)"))
 (segment (start 168.225 79.975) (end 168.225 82.125) (width 0.2) (layer "F.Cu") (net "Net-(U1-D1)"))
 (via (at 167.45 82.9) (size 0.6) (drill 0.3) (layers "F.Cu" "B.Cu") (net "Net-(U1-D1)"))
 (segment (start 167.45 82.9) (end 166.225 84.125) (width 0.2) (layer "B.Cu") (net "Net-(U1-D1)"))
 (segment (start 93.495 86.33) (end 79.67 86.33) (width 0.2) (layer "B.Cu") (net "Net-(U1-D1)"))
 (segment (start 131.75 85.92) (end 102.17 85.92) (width 0.2) (layer "B.Cu") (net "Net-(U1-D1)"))
 (segment (start 133.545 84.125) (end 131.75 85.92) (width 0.2) (layer "B.Cu") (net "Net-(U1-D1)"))
 (segment (start 102.17 85.92) (end 100.825 84.575) (width 0.2) (layer "B.Cu") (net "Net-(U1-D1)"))
 (segment (start 166.225 84.125) (end 133.545 84.125) (width 0.2) (layer "B.Cu") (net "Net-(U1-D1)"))
 (segment (start 95.25 84.575) (end 93.495 86.33) (width 0.2) (layer "B.Cu") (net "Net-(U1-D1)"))
 (segment (start 100.825 84.575) (end 95.25 84.575) (width 0.2) (layer "B.Cu") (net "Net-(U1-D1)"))
 (segment (start 70.575 76.275) (end 60.52 86.33) (width 0.2) (layer "F.Cu") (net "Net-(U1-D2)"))
 (segment (start 165.685 78.185) (end 163.775 76.275) (width 0.2) (layer "F.Cu") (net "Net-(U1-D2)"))
 (segment (start 165.685 79.975) (end 165.685 78.185) (width 0.2) (layer "F.Cu") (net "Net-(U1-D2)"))
 (segment (start 163.775 76.275) (end 70.575 76.275) (width 0.2) (layer "F.Cu") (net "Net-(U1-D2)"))
 (segment (start 72.425 76.725) (end 70.825 78.325) (width 0.2) (layer "F.Cu") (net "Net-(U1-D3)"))
 (segment (start 159.895 76.725) (end 72.425 76.725) (width 0.2) (layer "F.Cu") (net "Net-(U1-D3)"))
 (segment (start 163.145 79.975) (end 159.895 76.725) (width 0.2) (layer "F.Cu") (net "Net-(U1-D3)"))
 (via (at 70.825 78.325) (size 0.6) (drill 0.3) (layers "F.Cu" "B.Cu") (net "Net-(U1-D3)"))
 (segment (start 41.31 84.715) (end 45.225 80.8) (width 0.2) (layer "B.Cu") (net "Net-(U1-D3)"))
 (segment (start 70.825 78.325) (end 68.35 80.8) (width 0.2) (layer "B.Cu") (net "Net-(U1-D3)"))
 (segment (start 41.31 86.31) (end 41.31 84.715) (width 0.2) (layer "B.Cu") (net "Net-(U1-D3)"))
 (segment (start 68.35 80.8) (end 45.225 80.8) (width 0.2) (layer "B.Cu") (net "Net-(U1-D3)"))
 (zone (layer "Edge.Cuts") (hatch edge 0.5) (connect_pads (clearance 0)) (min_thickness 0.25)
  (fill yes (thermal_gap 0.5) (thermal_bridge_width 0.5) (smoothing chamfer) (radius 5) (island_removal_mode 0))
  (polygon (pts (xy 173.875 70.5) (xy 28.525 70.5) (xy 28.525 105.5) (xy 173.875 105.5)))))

